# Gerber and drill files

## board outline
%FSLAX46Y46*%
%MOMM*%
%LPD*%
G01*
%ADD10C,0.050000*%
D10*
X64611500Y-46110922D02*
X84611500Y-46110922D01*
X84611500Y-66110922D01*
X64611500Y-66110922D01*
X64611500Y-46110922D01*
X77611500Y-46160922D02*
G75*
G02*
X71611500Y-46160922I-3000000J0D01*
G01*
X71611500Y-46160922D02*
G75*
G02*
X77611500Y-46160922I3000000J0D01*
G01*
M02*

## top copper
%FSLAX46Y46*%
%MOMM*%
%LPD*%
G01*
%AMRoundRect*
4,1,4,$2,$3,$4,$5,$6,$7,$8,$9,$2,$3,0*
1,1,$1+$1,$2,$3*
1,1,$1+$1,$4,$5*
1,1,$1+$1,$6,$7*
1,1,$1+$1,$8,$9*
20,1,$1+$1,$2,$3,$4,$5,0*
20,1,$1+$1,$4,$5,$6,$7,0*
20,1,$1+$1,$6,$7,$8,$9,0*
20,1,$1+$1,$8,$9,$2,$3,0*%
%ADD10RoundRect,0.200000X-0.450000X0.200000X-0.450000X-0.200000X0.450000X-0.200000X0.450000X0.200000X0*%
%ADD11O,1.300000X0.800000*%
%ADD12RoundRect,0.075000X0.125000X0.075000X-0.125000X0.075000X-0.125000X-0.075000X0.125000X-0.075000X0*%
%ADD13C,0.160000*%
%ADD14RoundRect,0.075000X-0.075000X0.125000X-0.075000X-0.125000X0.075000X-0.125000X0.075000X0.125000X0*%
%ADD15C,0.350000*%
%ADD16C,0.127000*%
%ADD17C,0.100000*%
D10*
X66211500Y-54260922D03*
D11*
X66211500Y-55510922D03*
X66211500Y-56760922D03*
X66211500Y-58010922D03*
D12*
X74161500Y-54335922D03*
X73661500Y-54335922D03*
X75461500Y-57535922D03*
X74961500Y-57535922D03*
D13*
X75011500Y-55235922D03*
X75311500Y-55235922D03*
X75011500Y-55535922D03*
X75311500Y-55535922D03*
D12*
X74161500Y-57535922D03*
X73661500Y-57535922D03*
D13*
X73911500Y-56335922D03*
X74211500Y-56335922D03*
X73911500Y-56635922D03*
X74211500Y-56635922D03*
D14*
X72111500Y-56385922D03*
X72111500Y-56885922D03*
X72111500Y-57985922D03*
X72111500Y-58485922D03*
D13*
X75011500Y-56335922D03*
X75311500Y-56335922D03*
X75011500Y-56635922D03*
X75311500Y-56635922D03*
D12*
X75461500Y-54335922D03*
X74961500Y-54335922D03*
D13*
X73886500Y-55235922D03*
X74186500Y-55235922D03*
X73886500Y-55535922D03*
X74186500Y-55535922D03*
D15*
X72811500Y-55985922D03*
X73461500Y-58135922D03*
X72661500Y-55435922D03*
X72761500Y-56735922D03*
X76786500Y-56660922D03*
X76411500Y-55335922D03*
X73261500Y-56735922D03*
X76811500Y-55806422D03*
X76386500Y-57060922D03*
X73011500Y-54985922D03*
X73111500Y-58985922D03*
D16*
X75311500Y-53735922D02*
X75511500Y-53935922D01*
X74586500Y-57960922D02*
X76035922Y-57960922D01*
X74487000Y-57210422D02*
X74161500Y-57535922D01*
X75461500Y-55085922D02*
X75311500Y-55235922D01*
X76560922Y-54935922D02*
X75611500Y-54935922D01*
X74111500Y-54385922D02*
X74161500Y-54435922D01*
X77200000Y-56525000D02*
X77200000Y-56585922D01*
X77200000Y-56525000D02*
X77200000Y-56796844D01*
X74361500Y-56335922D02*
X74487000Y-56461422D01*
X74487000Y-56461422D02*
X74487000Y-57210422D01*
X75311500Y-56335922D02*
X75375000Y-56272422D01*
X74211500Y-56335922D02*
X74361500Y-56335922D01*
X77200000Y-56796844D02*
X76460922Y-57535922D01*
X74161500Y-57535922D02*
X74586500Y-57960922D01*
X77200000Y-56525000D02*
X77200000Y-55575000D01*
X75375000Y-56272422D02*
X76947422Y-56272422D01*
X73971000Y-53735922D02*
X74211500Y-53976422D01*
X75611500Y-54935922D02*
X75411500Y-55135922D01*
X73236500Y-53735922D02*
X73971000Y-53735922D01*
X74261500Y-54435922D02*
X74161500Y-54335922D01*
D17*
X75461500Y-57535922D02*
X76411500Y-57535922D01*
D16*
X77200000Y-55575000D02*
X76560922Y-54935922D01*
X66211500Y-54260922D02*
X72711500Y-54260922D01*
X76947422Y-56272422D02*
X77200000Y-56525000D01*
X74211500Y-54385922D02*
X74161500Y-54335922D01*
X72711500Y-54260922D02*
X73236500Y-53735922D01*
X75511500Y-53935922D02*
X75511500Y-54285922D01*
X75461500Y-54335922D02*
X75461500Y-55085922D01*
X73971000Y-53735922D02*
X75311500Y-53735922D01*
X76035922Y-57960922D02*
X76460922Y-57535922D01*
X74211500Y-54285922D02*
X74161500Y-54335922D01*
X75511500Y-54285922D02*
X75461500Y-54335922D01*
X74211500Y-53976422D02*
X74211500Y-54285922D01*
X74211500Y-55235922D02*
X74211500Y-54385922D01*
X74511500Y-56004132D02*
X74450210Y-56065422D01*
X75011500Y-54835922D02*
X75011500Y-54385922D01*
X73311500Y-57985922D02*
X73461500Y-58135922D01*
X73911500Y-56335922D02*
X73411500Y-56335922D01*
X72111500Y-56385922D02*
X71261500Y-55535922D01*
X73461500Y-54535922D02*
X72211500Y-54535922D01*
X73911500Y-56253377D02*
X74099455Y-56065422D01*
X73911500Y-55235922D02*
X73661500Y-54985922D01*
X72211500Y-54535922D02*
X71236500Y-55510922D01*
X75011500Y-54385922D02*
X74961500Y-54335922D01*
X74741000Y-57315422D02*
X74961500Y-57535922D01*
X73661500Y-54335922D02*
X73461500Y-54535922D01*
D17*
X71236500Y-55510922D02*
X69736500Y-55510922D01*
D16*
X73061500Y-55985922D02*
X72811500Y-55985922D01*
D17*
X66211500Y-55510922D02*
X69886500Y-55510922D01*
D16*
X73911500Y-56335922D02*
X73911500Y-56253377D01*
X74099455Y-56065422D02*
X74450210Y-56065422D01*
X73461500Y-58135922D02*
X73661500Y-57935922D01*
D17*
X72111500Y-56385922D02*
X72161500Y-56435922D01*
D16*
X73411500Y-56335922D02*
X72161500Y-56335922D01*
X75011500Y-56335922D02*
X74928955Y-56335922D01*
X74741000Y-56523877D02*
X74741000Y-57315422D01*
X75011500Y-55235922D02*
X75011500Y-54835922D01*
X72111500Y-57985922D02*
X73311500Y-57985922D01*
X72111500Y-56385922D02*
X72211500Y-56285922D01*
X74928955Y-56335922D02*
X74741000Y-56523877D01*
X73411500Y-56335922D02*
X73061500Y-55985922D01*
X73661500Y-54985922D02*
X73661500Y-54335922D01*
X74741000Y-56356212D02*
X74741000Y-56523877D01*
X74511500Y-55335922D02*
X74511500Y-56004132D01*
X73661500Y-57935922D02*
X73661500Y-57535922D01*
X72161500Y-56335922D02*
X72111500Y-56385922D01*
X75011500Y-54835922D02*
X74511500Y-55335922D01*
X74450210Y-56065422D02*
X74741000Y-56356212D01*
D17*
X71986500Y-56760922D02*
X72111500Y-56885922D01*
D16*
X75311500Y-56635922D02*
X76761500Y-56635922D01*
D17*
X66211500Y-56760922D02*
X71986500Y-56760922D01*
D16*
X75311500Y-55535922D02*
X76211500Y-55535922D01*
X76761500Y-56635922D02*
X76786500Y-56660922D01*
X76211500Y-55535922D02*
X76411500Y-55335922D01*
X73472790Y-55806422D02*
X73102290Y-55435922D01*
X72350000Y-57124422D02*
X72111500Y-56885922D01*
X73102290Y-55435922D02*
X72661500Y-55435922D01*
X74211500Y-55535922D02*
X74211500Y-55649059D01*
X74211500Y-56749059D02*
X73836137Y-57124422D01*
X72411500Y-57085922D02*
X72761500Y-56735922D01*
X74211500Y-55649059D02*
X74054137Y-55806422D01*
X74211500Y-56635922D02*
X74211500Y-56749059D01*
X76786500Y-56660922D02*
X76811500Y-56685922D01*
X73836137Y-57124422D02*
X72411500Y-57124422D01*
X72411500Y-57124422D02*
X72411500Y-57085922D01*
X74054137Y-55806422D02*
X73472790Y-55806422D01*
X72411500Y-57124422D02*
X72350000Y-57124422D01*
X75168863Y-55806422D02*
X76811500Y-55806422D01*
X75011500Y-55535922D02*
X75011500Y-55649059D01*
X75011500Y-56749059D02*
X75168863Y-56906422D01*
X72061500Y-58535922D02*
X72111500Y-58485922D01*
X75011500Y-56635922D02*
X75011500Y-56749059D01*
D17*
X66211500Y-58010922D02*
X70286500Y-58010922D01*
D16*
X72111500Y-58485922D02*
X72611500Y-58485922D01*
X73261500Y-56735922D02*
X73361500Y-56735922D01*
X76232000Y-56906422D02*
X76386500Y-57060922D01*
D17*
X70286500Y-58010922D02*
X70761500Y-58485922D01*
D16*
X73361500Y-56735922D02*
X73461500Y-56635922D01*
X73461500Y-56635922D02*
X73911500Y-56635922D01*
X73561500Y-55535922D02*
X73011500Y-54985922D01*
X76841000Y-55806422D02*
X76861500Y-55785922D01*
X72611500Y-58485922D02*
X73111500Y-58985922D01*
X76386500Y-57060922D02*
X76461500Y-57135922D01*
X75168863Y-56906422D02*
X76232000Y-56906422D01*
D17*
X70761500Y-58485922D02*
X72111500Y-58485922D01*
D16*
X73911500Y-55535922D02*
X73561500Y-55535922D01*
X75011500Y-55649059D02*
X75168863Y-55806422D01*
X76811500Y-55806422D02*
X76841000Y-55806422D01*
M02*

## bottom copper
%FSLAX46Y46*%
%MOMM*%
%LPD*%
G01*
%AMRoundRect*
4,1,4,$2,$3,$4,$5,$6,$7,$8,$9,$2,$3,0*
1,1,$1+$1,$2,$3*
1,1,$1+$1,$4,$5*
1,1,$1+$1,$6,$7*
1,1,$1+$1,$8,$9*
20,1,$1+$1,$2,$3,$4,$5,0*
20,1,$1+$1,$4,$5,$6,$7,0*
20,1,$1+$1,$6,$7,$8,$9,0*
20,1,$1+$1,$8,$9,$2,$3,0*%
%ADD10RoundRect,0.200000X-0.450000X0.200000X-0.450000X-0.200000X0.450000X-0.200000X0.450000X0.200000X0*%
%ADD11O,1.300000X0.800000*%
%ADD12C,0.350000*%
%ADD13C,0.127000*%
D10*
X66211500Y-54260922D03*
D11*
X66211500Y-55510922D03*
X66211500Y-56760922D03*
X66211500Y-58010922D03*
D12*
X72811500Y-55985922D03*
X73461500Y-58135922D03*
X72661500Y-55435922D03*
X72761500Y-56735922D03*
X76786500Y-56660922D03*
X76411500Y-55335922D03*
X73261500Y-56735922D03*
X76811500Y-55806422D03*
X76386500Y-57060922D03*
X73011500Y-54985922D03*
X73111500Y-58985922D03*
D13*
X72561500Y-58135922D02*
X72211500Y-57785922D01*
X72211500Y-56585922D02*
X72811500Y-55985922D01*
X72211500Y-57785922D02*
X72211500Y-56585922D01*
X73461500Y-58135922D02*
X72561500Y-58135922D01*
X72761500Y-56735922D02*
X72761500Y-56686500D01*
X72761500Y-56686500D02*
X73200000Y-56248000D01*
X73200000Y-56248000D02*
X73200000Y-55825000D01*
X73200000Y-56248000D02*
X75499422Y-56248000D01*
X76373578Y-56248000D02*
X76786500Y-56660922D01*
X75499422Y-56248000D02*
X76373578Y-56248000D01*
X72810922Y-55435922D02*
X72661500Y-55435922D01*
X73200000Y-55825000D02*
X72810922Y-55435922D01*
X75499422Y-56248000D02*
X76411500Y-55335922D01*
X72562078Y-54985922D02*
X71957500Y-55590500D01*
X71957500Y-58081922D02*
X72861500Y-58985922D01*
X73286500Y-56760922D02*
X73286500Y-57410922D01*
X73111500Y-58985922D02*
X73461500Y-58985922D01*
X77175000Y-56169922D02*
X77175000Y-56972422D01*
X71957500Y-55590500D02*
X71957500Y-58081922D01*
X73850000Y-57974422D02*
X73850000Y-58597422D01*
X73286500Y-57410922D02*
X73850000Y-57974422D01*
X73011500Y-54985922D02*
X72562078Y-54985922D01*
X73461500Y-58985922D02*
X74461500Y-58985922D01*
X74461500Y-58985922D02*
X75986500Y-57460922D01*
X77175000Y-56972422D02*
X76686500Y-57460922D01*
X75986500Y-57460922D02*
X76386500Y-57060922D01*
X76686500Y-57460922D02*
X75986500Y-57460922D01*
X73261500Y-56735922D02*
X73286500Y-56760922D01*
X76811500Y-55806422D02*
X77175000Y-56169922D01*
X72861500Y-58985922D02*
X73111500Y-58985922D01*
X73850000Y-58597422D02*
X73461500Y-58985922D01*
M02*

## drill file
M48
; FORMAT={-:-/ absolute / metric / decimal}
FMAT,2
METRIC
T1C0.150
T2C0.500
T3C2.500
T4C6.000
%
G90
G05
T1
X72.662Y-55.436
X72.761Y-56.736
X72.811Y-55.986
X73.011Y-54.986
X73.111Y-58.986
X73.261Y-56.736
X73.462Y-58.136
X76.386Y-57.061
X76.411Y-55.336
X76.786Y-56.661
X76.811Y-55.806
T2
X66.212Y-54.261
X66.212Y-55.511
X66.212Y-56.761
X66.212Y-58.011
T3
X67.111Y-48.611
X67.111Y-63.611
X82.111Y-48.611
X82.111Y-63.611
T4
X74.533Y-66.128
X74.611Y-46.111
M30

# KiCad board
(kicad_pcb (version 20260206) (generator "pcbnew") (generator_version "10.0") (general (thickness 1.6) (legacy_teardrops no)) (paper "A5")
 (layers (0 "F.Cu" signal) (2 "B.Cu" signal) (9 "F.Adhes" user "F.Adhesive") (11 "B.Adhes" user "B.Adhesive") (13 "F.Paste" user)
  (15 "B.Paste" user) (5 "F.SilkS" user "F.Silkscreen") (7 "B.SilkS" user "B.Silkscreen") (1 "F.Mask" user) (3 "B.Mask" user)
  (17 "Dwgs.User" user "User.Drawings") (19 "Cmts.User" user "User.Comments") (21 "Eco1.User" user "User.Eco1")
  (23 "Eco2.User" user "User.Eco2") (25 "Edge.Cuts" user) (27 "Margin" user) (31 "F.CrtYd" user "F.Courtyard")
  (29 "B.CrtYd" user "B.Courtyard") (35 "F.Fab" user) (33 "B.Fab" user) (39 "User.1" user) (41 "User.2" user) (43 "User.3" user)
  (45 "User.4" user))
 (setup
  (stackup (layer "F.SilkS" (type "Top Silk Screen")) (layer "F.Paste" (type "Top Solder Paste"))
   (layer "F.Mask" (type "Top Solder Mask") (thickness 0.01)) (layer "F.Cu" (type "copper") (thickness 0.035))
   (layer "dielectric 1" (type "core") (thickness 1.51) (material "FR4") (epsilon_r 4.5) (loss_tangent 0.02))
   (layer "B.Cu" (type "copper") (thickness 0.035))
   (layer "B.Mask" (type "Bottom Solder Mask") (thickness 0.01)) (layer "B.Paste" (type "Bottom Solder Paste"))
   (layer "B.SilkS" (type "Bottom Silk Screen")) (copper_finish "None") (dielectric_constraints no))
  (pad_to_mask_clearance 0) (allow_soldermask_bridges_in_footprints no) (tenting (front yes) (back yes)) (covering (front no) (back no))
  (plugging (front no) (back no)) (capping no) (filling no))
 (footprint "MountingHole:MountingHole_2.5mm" (layer "F.Cu") (at 67.1115 48.610922)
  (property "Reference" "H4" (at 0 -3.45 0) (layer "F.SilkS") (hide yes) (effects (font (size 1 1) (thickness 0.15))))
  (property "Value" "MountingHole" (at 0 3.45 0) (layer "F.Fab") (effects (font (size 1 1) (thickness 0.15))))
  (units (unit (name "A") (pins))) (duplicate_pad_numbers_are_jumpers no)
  (pad "" np_thru_hole circle (at 0 0) (size 2.5 2.5) (drill 2.5) (layers "*.Cu" "*.Mask")))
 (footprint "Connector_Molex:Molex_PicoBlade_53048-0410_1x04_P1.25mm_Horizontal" (layer "F.Cu") (at 66.2115 54.260922 -90)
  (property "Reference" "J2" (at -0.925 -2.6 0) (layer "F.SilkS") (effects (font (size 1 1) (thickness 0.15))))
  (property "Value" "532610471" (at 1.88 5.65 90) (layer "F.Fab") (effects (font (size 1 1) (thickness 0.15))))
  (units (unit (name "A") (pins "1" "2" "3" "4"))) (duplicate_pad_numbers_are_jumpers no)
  (pad "1" thru_hole roundrect (at 0 0 270) (size 0.8 1.3) (drill 0.5) (layers "*.Cu" "*.Mask") (remove_unused_layers no)
   (roundrect_rratio 0.25) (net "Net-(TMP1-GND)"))
  (pad "2" thru_hole oval (at 1.25 0 270) (size 0.8 1.3) (drill 0.5) (layers "*.Cu" "*.Mask") (remove_unused_layers no)
   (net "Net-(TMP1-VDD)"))
  (pad "3" thru_hole oval (at 2.5 0 270) (size 0.8 1.3) (drill 0.5) (layers "*.Cu" "*.Mask") (remove_unused_layers no)
   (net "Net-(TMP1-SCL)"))
  (pad "4" thru_hole oval (at 3.75 0 270) (size 0.8 1.3) (drill 0.5) (layers "*.Cu" "*.Mask") (remove_unused_layers no)
   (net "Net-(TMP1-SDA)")))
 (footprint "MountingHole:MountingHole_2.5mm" (layer "F.Cu") (at 82.1115 63.610922)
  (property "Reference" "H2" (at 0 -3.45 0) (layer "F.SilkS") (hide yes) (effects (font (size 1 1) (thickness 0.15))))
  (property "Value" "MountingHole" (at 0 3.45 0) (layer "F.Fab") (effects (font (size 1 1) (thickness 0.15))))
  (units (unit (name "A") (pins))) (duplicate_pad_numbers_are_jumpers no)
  (pad "" np_thru_hole circle (at 0 0) (size 2.5 2.5) (drill 2.5) (layers "*.Cu" "*.Mask")))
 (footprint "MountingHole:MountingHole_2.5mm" (layer "F.Cu") (at 82.1115 48.610922)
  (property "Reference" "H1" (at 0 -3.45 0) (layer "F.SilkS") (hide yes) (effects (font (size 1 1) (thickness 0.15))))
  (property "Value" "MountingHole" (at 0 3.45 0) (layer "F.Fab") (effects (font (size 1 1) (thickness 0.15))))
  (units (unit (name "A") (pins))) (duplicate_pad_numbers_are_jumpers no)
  (pad "" np_thru_hole circle (at 0 0) (size 2.5 2.5) (drill 2.5) (layers "*.Cu" "*.Mask")))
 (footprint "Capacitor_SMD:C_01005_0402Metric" (layer "F.Cu") (at 73.9115 54.335922 180)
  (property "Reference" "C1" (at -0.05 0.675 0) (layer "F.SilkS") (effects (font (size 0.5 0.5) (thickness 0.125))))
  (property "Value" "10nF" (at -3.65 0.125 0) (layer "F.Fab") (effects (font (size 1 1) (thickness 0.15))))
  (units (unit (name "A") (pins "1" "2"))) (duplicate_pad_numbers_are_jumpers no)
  (pad "" smd roundrect (at -0.275 0 180) (size 0.27 0.27) (layers "F.Paste") (roundrect_rratio 0.25))
  (pad "" smd roundrect (at 0.275 0 180) (size 0.27 0.27) (layers "F.Paste") (roundrect_rratio 0.25))
  (pad "1" smd roundrect (at -0.25 0 180) (size 0.4 0.3) (layers "F.Cu" "F.Mask") (roundrect_rratio 0.25) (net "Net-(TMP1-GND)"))
  (pad "2" smd roundrect (at 0.25 0 180) (size 0.4 0.3) (layers "F.Cu" "F.Mask") (roundrect_rratio 0.25) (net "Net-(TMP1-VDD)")))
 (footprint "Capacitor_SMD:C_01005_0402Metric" (layer "F.Cu") (at 75.2115 57.535922 180)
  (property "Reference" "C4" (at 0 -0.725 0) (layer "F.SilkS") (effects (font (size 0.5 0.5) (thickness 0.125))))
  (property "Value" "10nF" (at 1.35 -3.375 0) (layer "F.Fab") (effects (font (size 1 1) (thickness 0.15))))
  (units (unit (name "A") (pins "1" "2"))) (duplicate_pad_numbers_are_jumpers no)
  (pad "" smd roundrect (at -0.275 0 180) (size 0.27 0.27) (layers "F.Paste") (roundrect_rratio 0.25))
  (pad "" smd roundrect (at 0.275 0 180) (size 0.27 0.27) (layers "F.Paste") (roundrect_rratio 0.25))
  (pad "1" smd roundrect (at -0.25 0 180) (size 0.4 0.3) (layers "F.Cu" "F.Mask") (roundrect_rratio 0.25) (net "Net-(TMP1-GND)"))
  (pad "2" smd roundrect (at 0.25 0 180) (size 0.4 0.3) (layers "F.Cu" "F.Mask") (roundrect_rratio 0.25) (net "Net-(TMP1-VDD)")))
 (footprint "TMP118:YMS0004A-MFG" (layer "F.Cu") (at 75.1615 55.385922)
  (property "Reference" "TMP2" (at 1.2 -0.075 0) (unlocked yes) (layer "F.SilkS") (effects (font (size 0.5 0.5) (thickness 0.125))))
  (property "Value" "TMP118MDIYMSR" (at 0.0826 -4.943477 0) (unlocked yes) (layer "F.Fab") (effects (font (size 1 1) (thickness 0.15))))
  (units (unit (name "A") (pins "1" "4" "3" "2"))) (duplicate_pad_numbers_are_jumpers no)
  (pad "1" smd circle (at -0.15 -0.15) (size 0.16 0.16) (layers "F.Cu" "F.Mask") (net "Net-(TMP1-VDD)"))
  (pad "2" smd circle (at 0.15 -0.15) (size 0.16 0.16) (layers "F.Cu" "F.Mask") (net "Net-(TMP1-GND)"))
  (pad "3" smd circle (at -0.15 0.15) (size 0.16 0.16) (layers "F.Cu" "F.Mask") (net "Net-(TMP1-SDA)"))
  (pad "4" smd circle (at 0.15 0.15) (size 0.16 0.16) (layers "F.Cu" "F.Mask") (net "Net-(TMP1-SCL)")))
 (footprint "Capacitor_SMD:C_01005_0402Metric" (layer "F.Cu") (at 73.9115 57.535922 180)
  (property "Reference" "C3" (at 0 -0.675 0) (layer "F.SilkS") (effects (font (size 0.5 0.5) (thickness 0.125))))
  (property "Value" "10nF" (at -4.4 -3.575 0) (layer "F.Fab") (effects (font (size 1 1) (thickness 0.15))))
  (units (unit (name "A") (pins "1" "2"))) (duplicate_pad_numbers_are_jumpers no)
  (pad "" smd roundrect (at -0.275 0 180) (size 0.27 0.27) (layers "F.Paste") (roundrect_rratio 0.25))
  (pad "" smd roundrect (at 0.275 0 180) (size 0.27 0.27) (layers "F.Paste") (roundrect_rratio 0.25))
  (pad "1" smd roundrect (at -0.25 0 180) (size 0.4 0.3) (layers "F.Cu" "F.Mask") (roundrect_rratio 0.25) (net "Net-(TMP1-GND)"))
  (pad "2" smd roundrect (at 0.25 0 180) (size 0.4 0.3) (layers "F.Cu" "F.Mask") (roundrect_rratio 0.25) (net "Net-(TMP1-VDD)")))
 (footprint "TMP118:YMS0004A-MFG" (layer "F.Cu") (at 74.0615 56.485922)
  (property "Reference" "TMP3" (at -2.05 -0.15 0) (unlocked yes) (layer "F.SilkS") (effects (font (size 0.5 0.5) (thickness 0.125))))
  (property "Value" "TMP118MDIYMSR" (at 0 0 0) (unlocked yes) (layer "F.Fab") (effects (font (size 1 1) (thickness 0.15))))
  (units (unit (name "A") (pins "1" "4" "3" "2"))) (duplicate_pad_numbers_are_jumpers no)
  (pad "1" smd circle (at -0.15 -0.15) (size 0.16 0.16) (layers "F.Cu" "F.Mask") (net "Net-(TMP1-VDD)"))
  (pad "2" smd circle (at 0.15 -0.15) (size 0.16 0.16) (layers "F.Cu" "F.Mask") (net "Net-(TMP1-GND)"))
  (pad "3" smd circle (at -0.15 0.15) (size 0.16 0.16) (layers "F.Cu" "F.Mask") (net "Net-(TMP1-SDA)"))
  (pad "4" smd circle (at 0.15 0.15) (size 0.16 0.16) (layers "F.Cu" "F.Mask") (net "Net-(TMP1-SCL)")))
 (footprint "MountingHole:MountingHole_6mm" (layer "F.Cu") (at 74.6115 46.110922)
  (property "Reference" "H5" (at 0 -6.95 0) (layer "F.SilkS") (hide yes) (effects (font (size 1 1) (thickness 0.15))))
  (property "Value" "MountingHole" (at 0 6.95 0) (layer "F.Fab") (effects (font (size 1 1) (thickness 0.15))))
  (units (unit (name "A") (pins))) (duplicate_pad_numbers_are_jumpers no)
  (pad "" np_thru_hole circle (at 0 0) (size 6 6) (drill 6) (layers "*.Cu" "*.Mask")))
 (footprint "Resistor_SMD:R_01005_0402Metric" (layer "F.Cu") (at 72.1115 56.635922 -90)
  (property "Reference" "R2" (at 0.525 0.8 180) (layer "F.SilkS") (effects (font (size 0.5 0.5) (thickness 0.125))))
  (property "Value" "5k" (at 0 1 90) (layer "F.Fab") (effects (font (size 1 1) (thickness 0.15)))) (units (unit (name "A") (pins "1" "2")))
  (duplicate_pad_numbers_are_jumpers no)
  (pad "" smd roundrect (at -0.275 0 270) (size 0.27 0.27) (layers "F.Paste") (roundrect_rratio 0.25))
  (pad "" smd roundrect (at 0.275 0 270) (size 0.27 0.27) (layers "F.Paste") (roundrect_rratio 0.25))
  (pad "1" smd roundrect (at -0.25 0 270) (size 0.4 0.3) (layers "F.Cu" "F.Mask") (roundrect_rratio 0.25) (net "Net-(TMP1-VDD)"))
  (pad "2" smd roundrect (at 0.25 0 270) (size 0.4 0.3) (layers "F.Cu" "F.Mask") (roundrect_rratio 0.25) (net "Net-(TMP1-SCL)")))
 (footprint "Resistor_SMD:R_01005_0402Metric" (layer "F.Cu") (at 72.1115 58.235922 -90)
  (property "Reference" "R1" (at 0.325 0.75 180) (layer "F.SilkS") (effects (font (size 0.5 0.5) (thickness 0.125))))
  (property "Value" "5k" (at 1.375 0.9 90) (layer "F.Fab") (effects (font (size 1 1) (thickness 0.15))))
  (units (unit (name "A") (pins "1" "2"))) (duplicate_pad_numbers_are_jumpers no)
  (pad "" smd roundrect (at -0.275 0 270) (size 0.27 0.27) (layers "F.Paste") (roundrect_rratio 0.25))
  (pad "" smd roundrect (at 0.275 0 270) (size 0.27 0.27) (layers "F.Paste") (roundrect_rratio 0.25))
  (pad "1" smd roundrect (at -0.25 0 270) (size 0.4 0.3) (layers "F.Cu" "F.Mask") (roundrect_rratio 0.25) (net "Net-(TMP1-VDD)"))
  (pad "2" smd roundrect (at 0.25 0 270) (size 0.4 0.3) (layers "F.Cu" "F.Mask") (roundrect_rratio 0.25) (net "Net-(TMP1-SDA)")))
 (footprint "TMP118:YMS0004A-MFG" (layer "F.Cu") (at 75.1615 56.485922)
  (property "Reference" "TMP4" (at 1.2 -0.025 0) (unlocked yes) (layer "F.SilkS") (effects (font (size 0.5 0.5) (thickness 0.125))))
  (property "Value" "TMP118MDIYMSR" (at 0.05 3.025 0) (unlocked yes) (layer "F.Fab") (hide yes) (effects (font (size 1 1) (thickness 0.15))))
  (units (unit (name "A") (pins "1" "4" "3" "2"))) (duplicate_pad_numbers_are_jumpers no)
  (pad "1" smd circle (at -0.15 -0.15) (size 0.16 0.16) (layers "F.Cu" "F.Mask") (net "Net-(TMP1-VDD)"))
  (pad "2" smd circle (at 0.15 -0.15) (size 0.16 0.16) (layers "F.Cu" "F.Mask") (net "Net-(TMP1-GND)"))
  (pad "3" smd circle (at -0.15 0.15) (size 0.16 0.16) (layers "F.Cu" "F.Mask") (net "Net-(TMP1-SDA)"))
  (pad "4" smd circle (at 0.15 0.15) (size 0.16 0.16) (layers "F.Cu" "F.Mask") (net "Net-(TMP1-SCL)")))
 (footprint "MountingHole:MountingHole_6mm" (layer "F.Cu") (at 74.532819 66.127741)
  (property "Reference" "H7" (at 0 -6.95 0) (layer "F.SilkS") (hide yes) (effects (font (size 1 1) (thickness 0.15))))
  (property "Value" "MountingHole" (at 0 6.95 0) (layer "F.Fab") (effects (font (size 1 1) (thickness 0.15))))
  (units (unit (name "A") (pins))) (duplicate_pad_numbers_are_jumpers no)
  (pad "" np_thru_hole circle (at 0 0) (size 6 6) (drill 6) (layers "*.Cu" "*.Mask")))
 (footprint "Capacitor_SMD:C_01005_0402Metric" (layer "F.Cu") (at 75.2115 54.335922 180)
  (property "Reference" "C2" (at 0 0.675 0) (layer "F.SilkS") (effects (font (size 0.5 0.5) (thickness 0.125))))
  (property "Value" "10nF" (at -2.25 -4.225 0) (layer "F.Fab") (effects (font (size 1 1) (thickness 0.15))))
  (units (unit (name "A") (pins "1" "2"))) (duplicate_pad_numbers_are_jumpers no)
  (pad "" smd roundrect (at -0.275 0 180) (size 0.27 0.27) (layers "F.Paste") (roundrect_rratio 0.25))
  (pad "" smd roundrect (at 0.275 0 180) (size 0.27 0.27) (layers "F.Paste") (roundrect_rratio 0.25))
  (pad "1" smd roundrect (at -0.25 0 180) (size 0.4 0.3) (layers "F.Cu" "F.Mask") (roundrect_rratio 0.25) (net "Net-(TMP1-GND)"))
  (pad "2" smd roundrect (at 0.25 0 180) (size 0.4 0.3) (layers "F.Cu" "F.Mask") (roundrect_rratio 0.25) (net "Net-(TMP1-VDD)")))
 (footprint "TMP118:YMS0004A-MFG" (layer "F.Cu") (at 74.0365 55.385922)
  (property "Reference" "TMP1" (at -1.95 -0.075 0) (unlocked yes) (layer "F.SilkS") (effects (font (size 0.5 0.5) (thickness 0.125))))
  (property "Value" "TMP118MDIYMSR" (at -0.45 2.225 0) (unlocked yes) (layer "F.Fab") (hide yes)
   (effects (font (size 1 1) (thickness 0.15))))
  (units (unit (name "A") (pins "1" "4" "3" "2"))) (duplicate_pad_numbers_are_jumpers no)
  (pad "1" smd circle (at -0.15 -0.15) (size 0.16 0.16) (layers "F.Cu" "F.Mask") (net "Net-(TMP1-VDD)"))
  (pad "2" smd circle (at 0.15 -0.15) (size 0.16 0.16) (layers "F.Cu" "F.Mask") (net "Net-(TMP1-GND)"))
  (pad "3" smd circle (at -0.15 0.15) (size 0.16 0.16) (layers "F.Cu" "F.Mask") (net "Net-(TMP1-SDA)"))
  (pad "4" smd circle (at 0.15 0.15) (size 0.16 0.16) (layers "F.Cu" "F.Mask") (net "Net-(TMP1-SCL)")))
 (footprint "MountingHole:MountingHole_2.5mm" (layer "F.Cu") (at 67.1115 63.610922)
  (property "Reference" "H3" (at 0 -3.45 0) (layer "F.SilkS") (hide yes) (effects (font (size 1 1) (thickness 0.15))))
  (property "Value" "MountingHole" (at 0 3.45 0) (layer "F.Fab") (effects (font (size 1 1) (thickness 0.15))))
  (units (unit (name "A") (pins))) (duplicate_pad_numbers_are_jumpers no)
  (pad "" np_thru_hole circle (at 0 0) (size 2.5 2.5) (drill 2.5) (layers "*.Cu" "*.Mask")))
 (gr_rect (start 64.6115 46.110922) (end 84.6115 66.110922) (stroke (width 0.05) (type solid)) (fill no) (layer "Edge.Cuts"))
 (gr_circle (center 74.6115 46.160922) (end 77.6115 46.160922) (stroke (width 0.05) (type default)) (fill no) (layer "Edge.Cuts"))
 (segment (start 75.3115 53.735922) (end 75.5115 53.935922) (width 0.127) (layer "F.Cu") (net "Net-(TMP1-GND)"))
 (segment (start 74.5865 57.960922) (end 76.035922 57.960922) (width 0.127) (layer "F.Cu") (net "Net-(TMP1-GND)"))
 (segment (start 74.487 57.210422) (end 74.1615 57.535922) (width 0.127) (layer "F.Cu") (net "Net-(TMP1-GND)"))
 (segment (start 75.4615 55.085922) (end 75.3115 55.235922) (width 0.127) (layer "F.Cu") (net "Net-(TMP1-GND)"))
 (segment (start 76.560922 54.935922) (end 75.6115 54.935922) (width 0.127) (layer "F.Cu") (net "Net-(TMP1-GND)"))
 (segment (start 74.1115 54.385922) (end 74.1615 54.435922) (width 0.127) (layer "F.Cu") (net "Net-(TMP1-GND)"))
 (segment (start 77.2 56.525) (end 77.2 56.585922) (width 0.127) (layer "F.Cu") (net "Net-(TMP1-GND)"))
 (segment (start 77.2 56.525) (end 77.2 56.796844) (width 0.127) (layer "F.Cu") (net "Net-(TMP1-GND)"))
 (segment (start 74.3615 56.335922) (end 74.487 56.461422) (width 0.127) (layer "F.Cu") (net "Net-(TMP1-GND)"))
 (segment (start 74.487 56.461422) (end 74.487 57.210422) (width 0.127) (layer "F.Cu") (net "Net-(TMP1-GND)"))
 (segment (start 75.3115 56.335922) (end 75.375 56.272422) (width 0.127) (layer "F.Cu") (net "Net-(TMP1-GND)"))
 (segment (start 74.2115 56.335922) (end 74.3615 56.335922) (width 0.127) (layer "F.Cu") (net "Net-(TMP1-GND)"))
 (segment (start 77.2 56.796844) (end 76.460922 57.535922) (width 0.127) (layer "F.Cu") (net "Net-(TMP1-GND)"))
 (segment (start 74.1615 57.535922) (end 74.5865 57.960922) (width 0.127) (layer "F.Cu") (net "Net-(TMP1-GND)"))
 (segment (start 77.2 56.525) (end 77.2 55.575) (width 0.127) (layer "F.Cu") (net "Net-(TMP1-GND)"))
 (segment (start 75.375 56.272422) (end 76.947422 56.272422) (width 0.127) (layer "F.Cu") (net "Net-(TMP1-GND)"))
 (segment (start 73.971 53.735922) (end 74.2115 53.976422) (width 0.127) (layer "F.Cu") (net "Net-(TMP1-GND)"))
 (segment (start 75.6115 54.935922) (end 75.4115 55.135922) (width 0.127) (layer "F.Cu") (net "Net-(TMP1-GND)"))
 (segment (start 73.2365 53.735922) (end 73.971 53.735922) (width 0.127) (layer "F.Cu") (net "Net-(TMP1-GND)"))
 (segment (start 74.2615 54.435922) (end 74.1615 54.335922) (width 0.127) (layer "F.Cu") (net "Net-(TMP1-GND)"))
 (segment (start 75.4615 57.535922) (end 76.4115 57.535922) (width 0.1) (layer "F.Cu") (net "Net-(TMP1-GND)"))
 (segment (start 77.2 55.575) (end 76.560922 54.935922) (width 0.127) (layer "F.Cu") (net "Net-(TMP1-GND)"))
 (segment (start 66.2115 54.260922) (end 72.7115 54.260922) (width 0.127) (layer "F.Cu") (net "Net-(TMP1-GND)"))
 (segment (start 76.947422 56.272422) (end 77.2 56.525) (width 0.127) (layer "F.Cu") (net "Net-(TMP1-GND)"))
 (segment (start 74.2115 54.385922) (end 74.1615 54.335922) (width 0.127) (layer "F.Cu") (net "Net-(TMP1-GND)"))
 (segment (start 72.7115 54.260922) (end 73.2365 53.735922) (width 0.127) (layer "F.Cu") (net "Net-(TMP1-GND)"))
 (segment (start 75.5115 53.935922) (end 75.5115 54.285922) (width 0.127) (layer "F.Cu") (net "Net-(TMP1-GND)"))
 (segment (start 75.4615 54.335922) (end 75.4615 55.085922) (width 0.127) (layer "F.Cu") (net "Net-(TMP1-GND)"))
 (segment (start 73.971 53.735922) (end 75.3115 53.735922) (width 0.127) (layer "F.Cu") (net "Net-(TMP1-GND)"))
 (segment (start 76.035922 57.960922) (end 76.460922 57.535922) (width 0.127) (layer "F.Cu") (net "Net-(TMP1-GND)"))
 (segment (start 74.2115 54.285922) (end 74.1615 54.335922) (width 0.127) (layer "F.Cu") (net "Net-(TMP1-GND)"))
 (segment (start 75.5115 54.285922) (end 75.4615 54.335922) (width 0.127) (layer "F.Cu") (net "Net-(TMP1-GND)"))
 (segment (start 74.2115 53.976422) (end 74.2115 54.285922) (width 0.127) (layer "F.Cu") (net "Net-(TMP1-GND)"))
 (segment (start 74.2115 55.235922) (end 74.2115 54.385922) (width 0.127) (layer "F.Cu") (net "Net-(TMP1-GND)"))
 (segment (start 74.5115 56.004132) (end 74.45021 56.065422) (width 0.127) (layer "F.Cu") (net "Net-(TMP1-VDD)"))
 (segment (start 75.0115 54.835922) (end 75.0115 54.385922) (width 0.127) (layer "F.Cu") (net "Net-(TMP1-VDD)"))
 (segment (start 73.3115 57.985922) (end 73.4615 58.135922) (width 0.127) (layer "F.Cu") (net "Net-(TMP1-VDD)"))
 (segment (start 73.9115 56.335922) (end 73.4115 56.335922) (width 0.127) (layer "F.Cu") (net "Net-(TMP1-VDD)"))
 (segment (start 72.1115 56.385922) (end 71.2615 55.535922) (width 0.127) (layer "F.Cu") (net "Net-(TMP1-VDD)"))
 (segment (start 73.4615 54.535922) (end 72.2115 54.535922) (width 0.127) (layer "F.Cu") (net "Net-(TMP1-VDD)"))
 (segment (start 73.9115 56.253377) (end 74.099455 56.065422) (width 0.127) (layer "F.Cu") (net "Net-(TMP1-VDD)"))
 (segment (start 73.9115 55.235922) (end 73.6615 54.985922) (width 0.127) (layer "F.Cu") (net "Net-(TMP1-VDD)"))
 (segment (start 72.2115 54.535922) (end 71.2365 55.510922) (width 0.127) (layer "F.Cu") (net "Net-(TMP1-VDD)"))
 (segment (start 75.0115 54.385922) (end 74.9615 54.335922) (width 0.127) (layer "F.Cu") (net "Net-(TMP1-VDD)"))
 (segment (start 74.741 57.315422) (end 74.9615 57.535922) (width 0.127) (layer "F.Cu") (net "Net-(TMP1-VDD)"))
 (segment (start 73.6615 54.335922) (end 73.4615 54.535922) (width 0.127) (layer "F.Cu") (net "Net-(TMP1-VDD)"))
 (segment (start 71.2365 55.510922) (end 69.7365 55.510922) (width 0.1) (layer "F.Cu") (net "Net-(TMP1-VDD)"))
 (segment (start 73.0615 55.985922) (end 72.8115 55.985922) (width 0.127) (layer "F.Cu") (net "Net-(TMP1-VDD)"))
 (segment (start 66.2115 55.510922) (end 69.8865 55.510922) (width 0.1) (layer "F.Cu") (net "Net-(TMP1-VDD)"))
 (segment (start 73.9115 56.335922) (end 73.9115 56.253377) (width 0.127) (layer "F.Cu") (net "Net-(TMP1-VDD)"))
 (segment (start 74.099455 56.065422) (end 74.45021 56.065422) (width 0.127) (layer "F.Cu") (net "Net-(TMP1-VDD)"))
 (segment (start 73.4615 58.135922) (end 73.6615 57.935922) (width 0.127) (layer "F.Cu") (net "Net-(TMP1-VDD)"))
 (segment (start 72.1115 56.385922) (end 72.1615 56.435922) (width 0.1) (layer "F.Cu") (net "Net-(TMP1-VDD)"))
 (segment (start 73.4115 56.335922) (end 72.1615 56.335922) (width 0.127) (layer "F.Cu") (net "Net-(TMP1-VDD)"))
 (segment (start 75.0115 56.335922) (end 74.928955 56.335922) (width 0.127) (layer "F.Cu") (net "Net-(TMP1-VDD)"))
 (segment (start 74.741 56.523877) (end 74.741 57.315422) (width 0.127) (layer "F.Cu") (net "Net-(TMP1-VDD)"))
 (segment (start 75.0115 55.235922) (end 75.0115 54.835922) (width 0.127) (layer "F.Cu") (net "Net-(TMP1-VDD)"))
 (segment (start 72.1115 57.985922) (end 73.3115 57.985922) (width 0.127) (layer "F.Cu") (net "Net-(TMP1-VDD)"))
 (segment (start 72.1115 56.385922) (end 72.2115 56.285922) (width 0.127) (layer "F.Cu") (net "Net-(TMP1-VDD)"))
 (segment (start 74.928955 56.335922) (end 74.741 56.523877) (width 0.127) (layer "F.Cu") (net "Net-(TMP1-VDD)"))
 (segment (start 73.4115 56.335922) (end 73.0615 55.985922) (width 0.127) (layer "F.Cu") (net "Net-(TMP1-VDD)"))
 (segment (start 73.6615 54.985922) (end 73.6615 54.335922) (width 0.127) (layer "F.Cu") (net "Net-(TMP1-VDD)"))
 (segment (start 74.741 56.356212) (end 74.741 56.523877) (width 0.127) (layer "F.Cu") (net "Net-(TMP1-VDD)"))
 (segment (start 74.5115 55.335922) (end 74.5115 56.004132) (width 0.127) (layer "F.Cu") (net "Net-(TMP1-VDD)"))
 (segment (start 73.6615 57.935922) (end 73.6615 57.535922) (width 0.127) (layer "F.Cu") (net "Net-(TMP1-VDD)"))
 (segment (start 72.1615 56.335922) (end 72.1115 56.385922) (width 0.127) (layer "F.Cu") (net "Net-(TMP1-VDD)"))
 (segment (start 75.0115 54.835922) (end 74.5115 55.335922) (width 0.127) (layer "F.Cu") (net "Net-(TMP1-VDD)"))
 (segment (start 74.45021 56.065422) (end 74.741 56.356212) (width 0.127) (layer "F.Cu") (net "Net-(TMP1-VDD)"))
 (via (at 72.8115 55.985922) (size 0.35) (drill 0.15) (layers "F.Cu" "B.Cu") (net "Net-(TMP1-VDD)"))
 (via (at 73.4615 58.135922) (size 0.35) (drill 0.15) (layers "F.Cu" "B.Cu") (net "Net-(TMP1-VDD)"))
 (segment (start 72.5615 58.135922) (end 72.2115 57.785922) (width 0.127) (layer "B.Cu") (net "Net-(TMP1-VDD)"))
 (segment (start 72.2115 56.585922) (end 72.8115 55.985922) (width 0.127) (layer "B.Cu") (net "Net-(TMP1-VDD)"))
 (segment (start 72.2115 57.785922) (end 72.2115 56.585922) (width 0.127) (layer "B.Cu") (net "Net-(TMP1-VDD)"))
 (segment (start 73.4615 58.135922) (end 72.5615 58.135922) (width 0.127) (layer "B.Cu") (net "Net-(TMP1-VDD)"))
 (segment (start 71.9865 56.760922) (end 72.1115 56.885922) (width 0.1) (layer "F.Cu") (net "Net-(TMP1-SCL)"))
 (segment (start 75.3115 56.635922) (end 76.7615 56.635922) (width 0.127) (layer "F.Cu") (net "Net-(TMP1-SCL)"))
 (segment (start 66.2115 56.760922) (end 71.9865 56.760922) (width 0.1) (layer "F.Cu") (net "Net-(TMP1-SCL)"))
 (segment (start 75.3115 55.535922) (end 76.2115 55.535922) (width 0.127) (layer "F.Cu") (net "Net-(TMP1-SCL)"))
 (segment (start 76.7615 56.635922) (end 76.7865 56.660922) (width 0.127) (layer "F.Cu") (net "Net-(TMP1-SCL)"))
 (segment (start 76.2115 55.535922) (end 76.4115 55.335922) (width 0.127) (layer "F.Cu") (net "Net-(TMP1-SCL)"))
 (segment (start 73.47279 55.806422) (end 73.10229 55.435922) (width 0.127) (layer "F.Cu") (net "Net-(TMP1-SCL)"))
 (segment (start 72.35 57.124422) (end 72.1115 56.885922) (width 0.127) (layer "F.Cu") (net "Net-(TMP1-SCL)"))
 (segment (start 73.10229 55.435922) (end 72.6615 55.435922) (width 0.127) (layer "F.Cu") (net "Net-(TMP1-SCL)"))
 (segment (start 74.2115 55.535922) (end 74.2115 55.649059) (width 0.127) (layer "F.Cu") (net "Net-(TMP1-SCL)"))
 (segment (start 74.2115 56.749059) (end 73.836137 57.124422) (width 0.127) (layer "F.Cu") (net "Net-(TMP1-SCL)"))
 (segment (start 72.4115 57.085922) (end 72.7615 56.735922) (width 0.127) (layer "F.Cu") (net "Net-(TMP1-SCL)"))
 (segment (start 74.2115 55.649059) (end 74.054137 55.806422) (width 0.127) (layer "F.Cu") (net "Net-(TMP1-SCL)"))
 (segment (start 74.2115 56.635922) (end 74.2115 56.749059) (width 0.127) (layer "F.Cu") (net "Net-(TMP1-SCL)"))
 (segment (start 76.7865 56.660922) (end 76.8115 56.685922) (width 0.127) (layer "F.Cu") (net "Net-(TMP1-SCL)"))
 (segment (start 73.836137 57.124422) (end 72.4115 57.124422) (width 0.127) (layer "F.Cu") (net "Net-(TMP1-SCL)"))
 (segment (start 72.4115 57.124422) (end 72.4115 57.085922) (width 0.127) (layer "F.Cu") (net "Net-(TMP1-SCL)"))
 (segment (start 74.054137 55.806422) (end 73.47279 55.806422) (width 0.127) (layer "F.Cu") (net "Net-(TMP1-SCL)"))
 (segment (start 72.4115 57.124422) (end 72.35 57.124422) (width 0.127) (layer "F.Cu") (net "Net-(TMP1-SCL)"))
 (via (at 72.6615 55.435922) (size 0.35) (drill 0.15) (layers "F.Cu" "B.Cu") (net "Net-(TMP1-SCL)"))
 (via (at 72.7615 56.735922) (size 0.35) (drill 0.15) (layers "F.Cu" "B.Cu") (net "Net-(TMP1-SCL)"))
 (via (at 76.7865 56.660922) (size 0.35) (drill 0.15) (layers "F.Cu" "B.Cu") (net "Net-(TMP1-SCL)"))
 (via (at 76.4115 55.335922) (size 0.35) (drill 0.15) (layers "F.Cu" "B.Cu") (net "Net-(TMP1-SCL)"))
 (segment (start 72.7615 56.735922) (end 72.7615 56.6865) (width 0.127) (layer "B.Cu") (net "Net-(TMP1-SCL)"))
 (segment (start 72.7615 56.6865) (end 73.2 56.248) (width 0.127) (layer "B.Cu") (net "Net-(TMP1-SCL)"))
 (segment (start 73.2 56.248) (end 73.2 55.825) (width 0.127) (layer "B.Cu") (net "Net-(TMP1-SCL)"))
 (segment (start 73.2 56.248) (end 75.499422 56.248) (width 0.127) (layer "B.Cu") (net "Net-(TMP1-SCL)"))
 (segment (start 76.373578 56.248) (end 76.7865 56.660922) (width 0.127) (layer "B.Cu") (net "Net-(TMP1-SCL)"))
 (segment (start 75.499422 56.248) (end 76.373578 56.248) (width 0.127) (layer "B.Cu") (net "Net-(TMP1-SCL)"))
 (segment (start 72.810922 55.435922) (end 72.6615 55.435922) (width 0.127) (layer "B.Cu") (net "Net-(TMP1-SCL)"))
 (segment (start 73.2 55.825) (end 72.810922 55.435922) (width 0.127) (layer "B.Cu") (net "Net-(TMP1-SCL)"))
 (segment (start 75.499422 56.248) (end 76.4115 55.335922) (width 0.127) (layer "B.Cu") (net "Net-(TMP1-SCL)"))
 (segment (start 75.168863 55.806422) (end 76.8115 55.806422) (width 0.127) (layer "F.Cu") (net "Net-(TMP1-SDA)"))
 (segment (start 75.0115 55.535922) (end 75.0115 55.649059) (width 0.127) (layer "F.Cu") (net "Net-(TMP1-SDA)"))
 (segment (start 75.0115 56.749059) (end 75.168863 56.906422) (width 0.127) (layer "F.Cu") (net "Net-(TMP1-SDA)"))
 (segment (start 72.0615 58.535922) (end 72.1115 58.485922) (width 0.127) (layer "F.Cu") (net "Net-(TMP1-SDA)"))
 (segment (start 75.0115 56.635922) (end 75.0115 56.749059) (width 0.127) (layer "F.Cu") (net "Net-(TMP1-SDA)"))
 (segment (start 66.2115 58.010922) (end 70.2865 58.010922) (width 0.1) (layer "F.Cu") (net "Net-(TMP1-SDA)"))
 (segment (start 72.1115 58.485922) (end 72.6115 58.485922) (width 0.127) (layer "F.Cu") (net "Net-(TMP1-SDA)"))
 (segment (start 73.2615 56.735922) (end 73.3615 56.735922) (width 0.127) (layer "F.Cu") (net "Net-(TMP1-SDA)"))
 (segment (start 76.232 56.906422) (end 76.3865 57.060922) (width 0.127) (layer "F.Cu") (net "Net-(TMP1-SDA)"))
 (segment (start 70.2865 58.010922) (end 70.7615 58.485922) (width 0.1) (layer "F.Cu") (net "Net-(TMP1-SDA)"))
 (segment (start 73.3615 56.735922) (end 73.4615 56.635922) (width 0.127) (layer "F.Cu") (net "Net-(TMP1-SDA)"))
 (segment (start 73.4615 56.635922) (end 73.9115 56.635922) (width 0.127) (layer "F.Cu") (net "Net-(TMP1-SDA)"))
 (segment (start 73.5615 55.535922) (end 73.0115 54.985922) (width 0.127) (layer "F.Cu") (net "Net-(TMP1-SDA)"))
 (segment (start 76.841 55.806422) (end 76.8615 55.785922) (width 0.127) (layer "F.Cu") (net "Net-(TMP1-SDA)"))
 (segment (start 72.6115 58.485922) (end 73.1115 58.985922) (width 0.127) (layer "F.Cu") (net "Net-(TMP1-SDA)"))
 (segment (start 76.3865 57.060922) (end 76.4615 57.135922) (width 0.127) (layer "F.Cu") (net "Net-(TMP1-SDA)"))
 (segment (start 75.168863 56.906422) (end 76.232 56.906422) (width 0.127) (layer "F.Cu") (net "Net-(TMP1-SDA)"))
 (segment (start 70.7615 58.485922) (end 72.1115 58.485922) (width 0.1) (layer "F.Cu") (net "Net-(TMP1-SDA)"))
 (segment (start 73.9115 55.535922) (end 73.5615 55.535922) (width 0.127) (layer "F.Cu") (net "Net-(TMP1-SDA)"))
 (segment (start 75.0115 55.649059) (end 75.168863 55.806422) (width 0.127) (layer "F.Cu") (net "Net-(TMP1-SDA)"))
 (segment (start 76.8115 55.806422) (end 76.841 55.806422) (width 0.127) (layer "F.Cu") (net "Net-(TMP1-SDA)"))
 (via (at 73.2615 56.735922) (size 0.35) (drill 0.15) (layers "F.Cu" "B.Cu") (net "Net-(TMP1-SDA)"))
 (via (at 76.8115 55.806422) (size 0.35) (drill 0.15) (layers "F.Cu" "B.Cu") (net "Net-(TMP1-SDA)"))
 (via (at 76.3865 57.060922) (size 0.35) (drill 0.15) (layers "F.Cu" "B.Cu") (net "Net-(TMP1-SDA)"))
 (via (at 73.0115 54.985922) (size 0.35) (drill 0.15) (layers "F.Cu" "B.Cu") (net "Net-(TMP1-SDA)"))
 (via (at 73.1115 58.985922) (size 0.35) (drill 0.15) (layers "F.Cu" "B.Cu") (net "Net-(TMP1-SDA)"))
 (segment (start 72.562078 54.985922) (end 71.9575 55.5905) (width 0.127) (layer "B.Cu") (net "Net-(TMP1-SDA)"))
 (segment (start 71.9575 58.081922) (end 72.8615 58.985922) (width 0.127) (layer "B.Cu") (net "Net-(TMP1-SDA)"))
 (segment (start 73.2865 56.760922) (end 73.2865 57.410922) (width 0.127) (layer "B.Cu") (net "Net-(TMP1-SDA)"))
 (segment (start 73.1115 58.985922) (end 73.4615 58.985922) (width 0.127) (layer "B.Cu") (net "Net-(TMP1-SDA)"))
 (segment (start 77.175 56.169922) (end 77.175 56.972422) (width 0.127) (layer "B.Cu") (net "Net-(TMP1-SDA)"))
 (segment (start 71.9575 55.5905) (end 71.9575 58.081922) (width 0.127) (layer "B.Cu") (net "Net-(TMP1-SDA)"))
 (segment (start 73.85 57.974422) (end 73.85 58.597422) (width 0.127) (layer "B.Cu") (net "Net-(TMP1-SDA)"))
 (segment (start 73.2865 57.410922) (end 73.85 57.974422) (width 0.127) (layer "B.Cu") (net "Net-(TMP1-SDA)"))
 (segment (start 73.0115 54.985922) (end 72.562078 54.985922) (width 0.127) (layer "B.Cu") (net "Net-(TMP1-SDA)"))
 (segment (start 73.4615 58.985922) (end 74.4615 58.985922) (width 0.127) (layer "B.Cu") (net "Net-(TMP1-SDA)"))
 (segment (start 74.4615 58.985922) (end 75.9865 57.460922) (width 0.127) (layer "B.Cu") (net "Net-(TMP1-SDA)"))
 (segment (start 77.175 56.972422) (end 76.6865 57.460922) (width 0.127) (layer "B.Cu") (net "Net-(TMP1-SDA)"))
 (segment (start 75.9865 57.460922) (end 76.3865 57.060922) (width 0.127) (layer "B.Cu") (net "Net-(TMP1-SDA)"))
 (segment (start 76.6865 57.460922) (end 75.9865 57.460922) (width 0.127) (layer "B.Cu") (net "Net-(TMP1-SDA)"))
 (segment (start 73.2615 56.735922) (end 73.2865 56.760922) (width 0.127) (layer "B.Cu") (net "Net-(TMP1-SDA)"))
 (segment (start 76.8115 55.806422) (end 77.175 56.169922) (width 0.127) (layer "B.Cu") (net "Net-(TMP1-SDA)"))
 (segment (start 72.8615 58.985922) (end 73.1115 58.985922) (width 0.127) (layer "B.Cu") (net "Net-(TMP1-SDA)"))
 (segment (start 73.85 58.597422) (end 73.4615 58.985922) (width 0.127) (layer "B.Cu") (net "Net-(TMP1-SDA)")))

